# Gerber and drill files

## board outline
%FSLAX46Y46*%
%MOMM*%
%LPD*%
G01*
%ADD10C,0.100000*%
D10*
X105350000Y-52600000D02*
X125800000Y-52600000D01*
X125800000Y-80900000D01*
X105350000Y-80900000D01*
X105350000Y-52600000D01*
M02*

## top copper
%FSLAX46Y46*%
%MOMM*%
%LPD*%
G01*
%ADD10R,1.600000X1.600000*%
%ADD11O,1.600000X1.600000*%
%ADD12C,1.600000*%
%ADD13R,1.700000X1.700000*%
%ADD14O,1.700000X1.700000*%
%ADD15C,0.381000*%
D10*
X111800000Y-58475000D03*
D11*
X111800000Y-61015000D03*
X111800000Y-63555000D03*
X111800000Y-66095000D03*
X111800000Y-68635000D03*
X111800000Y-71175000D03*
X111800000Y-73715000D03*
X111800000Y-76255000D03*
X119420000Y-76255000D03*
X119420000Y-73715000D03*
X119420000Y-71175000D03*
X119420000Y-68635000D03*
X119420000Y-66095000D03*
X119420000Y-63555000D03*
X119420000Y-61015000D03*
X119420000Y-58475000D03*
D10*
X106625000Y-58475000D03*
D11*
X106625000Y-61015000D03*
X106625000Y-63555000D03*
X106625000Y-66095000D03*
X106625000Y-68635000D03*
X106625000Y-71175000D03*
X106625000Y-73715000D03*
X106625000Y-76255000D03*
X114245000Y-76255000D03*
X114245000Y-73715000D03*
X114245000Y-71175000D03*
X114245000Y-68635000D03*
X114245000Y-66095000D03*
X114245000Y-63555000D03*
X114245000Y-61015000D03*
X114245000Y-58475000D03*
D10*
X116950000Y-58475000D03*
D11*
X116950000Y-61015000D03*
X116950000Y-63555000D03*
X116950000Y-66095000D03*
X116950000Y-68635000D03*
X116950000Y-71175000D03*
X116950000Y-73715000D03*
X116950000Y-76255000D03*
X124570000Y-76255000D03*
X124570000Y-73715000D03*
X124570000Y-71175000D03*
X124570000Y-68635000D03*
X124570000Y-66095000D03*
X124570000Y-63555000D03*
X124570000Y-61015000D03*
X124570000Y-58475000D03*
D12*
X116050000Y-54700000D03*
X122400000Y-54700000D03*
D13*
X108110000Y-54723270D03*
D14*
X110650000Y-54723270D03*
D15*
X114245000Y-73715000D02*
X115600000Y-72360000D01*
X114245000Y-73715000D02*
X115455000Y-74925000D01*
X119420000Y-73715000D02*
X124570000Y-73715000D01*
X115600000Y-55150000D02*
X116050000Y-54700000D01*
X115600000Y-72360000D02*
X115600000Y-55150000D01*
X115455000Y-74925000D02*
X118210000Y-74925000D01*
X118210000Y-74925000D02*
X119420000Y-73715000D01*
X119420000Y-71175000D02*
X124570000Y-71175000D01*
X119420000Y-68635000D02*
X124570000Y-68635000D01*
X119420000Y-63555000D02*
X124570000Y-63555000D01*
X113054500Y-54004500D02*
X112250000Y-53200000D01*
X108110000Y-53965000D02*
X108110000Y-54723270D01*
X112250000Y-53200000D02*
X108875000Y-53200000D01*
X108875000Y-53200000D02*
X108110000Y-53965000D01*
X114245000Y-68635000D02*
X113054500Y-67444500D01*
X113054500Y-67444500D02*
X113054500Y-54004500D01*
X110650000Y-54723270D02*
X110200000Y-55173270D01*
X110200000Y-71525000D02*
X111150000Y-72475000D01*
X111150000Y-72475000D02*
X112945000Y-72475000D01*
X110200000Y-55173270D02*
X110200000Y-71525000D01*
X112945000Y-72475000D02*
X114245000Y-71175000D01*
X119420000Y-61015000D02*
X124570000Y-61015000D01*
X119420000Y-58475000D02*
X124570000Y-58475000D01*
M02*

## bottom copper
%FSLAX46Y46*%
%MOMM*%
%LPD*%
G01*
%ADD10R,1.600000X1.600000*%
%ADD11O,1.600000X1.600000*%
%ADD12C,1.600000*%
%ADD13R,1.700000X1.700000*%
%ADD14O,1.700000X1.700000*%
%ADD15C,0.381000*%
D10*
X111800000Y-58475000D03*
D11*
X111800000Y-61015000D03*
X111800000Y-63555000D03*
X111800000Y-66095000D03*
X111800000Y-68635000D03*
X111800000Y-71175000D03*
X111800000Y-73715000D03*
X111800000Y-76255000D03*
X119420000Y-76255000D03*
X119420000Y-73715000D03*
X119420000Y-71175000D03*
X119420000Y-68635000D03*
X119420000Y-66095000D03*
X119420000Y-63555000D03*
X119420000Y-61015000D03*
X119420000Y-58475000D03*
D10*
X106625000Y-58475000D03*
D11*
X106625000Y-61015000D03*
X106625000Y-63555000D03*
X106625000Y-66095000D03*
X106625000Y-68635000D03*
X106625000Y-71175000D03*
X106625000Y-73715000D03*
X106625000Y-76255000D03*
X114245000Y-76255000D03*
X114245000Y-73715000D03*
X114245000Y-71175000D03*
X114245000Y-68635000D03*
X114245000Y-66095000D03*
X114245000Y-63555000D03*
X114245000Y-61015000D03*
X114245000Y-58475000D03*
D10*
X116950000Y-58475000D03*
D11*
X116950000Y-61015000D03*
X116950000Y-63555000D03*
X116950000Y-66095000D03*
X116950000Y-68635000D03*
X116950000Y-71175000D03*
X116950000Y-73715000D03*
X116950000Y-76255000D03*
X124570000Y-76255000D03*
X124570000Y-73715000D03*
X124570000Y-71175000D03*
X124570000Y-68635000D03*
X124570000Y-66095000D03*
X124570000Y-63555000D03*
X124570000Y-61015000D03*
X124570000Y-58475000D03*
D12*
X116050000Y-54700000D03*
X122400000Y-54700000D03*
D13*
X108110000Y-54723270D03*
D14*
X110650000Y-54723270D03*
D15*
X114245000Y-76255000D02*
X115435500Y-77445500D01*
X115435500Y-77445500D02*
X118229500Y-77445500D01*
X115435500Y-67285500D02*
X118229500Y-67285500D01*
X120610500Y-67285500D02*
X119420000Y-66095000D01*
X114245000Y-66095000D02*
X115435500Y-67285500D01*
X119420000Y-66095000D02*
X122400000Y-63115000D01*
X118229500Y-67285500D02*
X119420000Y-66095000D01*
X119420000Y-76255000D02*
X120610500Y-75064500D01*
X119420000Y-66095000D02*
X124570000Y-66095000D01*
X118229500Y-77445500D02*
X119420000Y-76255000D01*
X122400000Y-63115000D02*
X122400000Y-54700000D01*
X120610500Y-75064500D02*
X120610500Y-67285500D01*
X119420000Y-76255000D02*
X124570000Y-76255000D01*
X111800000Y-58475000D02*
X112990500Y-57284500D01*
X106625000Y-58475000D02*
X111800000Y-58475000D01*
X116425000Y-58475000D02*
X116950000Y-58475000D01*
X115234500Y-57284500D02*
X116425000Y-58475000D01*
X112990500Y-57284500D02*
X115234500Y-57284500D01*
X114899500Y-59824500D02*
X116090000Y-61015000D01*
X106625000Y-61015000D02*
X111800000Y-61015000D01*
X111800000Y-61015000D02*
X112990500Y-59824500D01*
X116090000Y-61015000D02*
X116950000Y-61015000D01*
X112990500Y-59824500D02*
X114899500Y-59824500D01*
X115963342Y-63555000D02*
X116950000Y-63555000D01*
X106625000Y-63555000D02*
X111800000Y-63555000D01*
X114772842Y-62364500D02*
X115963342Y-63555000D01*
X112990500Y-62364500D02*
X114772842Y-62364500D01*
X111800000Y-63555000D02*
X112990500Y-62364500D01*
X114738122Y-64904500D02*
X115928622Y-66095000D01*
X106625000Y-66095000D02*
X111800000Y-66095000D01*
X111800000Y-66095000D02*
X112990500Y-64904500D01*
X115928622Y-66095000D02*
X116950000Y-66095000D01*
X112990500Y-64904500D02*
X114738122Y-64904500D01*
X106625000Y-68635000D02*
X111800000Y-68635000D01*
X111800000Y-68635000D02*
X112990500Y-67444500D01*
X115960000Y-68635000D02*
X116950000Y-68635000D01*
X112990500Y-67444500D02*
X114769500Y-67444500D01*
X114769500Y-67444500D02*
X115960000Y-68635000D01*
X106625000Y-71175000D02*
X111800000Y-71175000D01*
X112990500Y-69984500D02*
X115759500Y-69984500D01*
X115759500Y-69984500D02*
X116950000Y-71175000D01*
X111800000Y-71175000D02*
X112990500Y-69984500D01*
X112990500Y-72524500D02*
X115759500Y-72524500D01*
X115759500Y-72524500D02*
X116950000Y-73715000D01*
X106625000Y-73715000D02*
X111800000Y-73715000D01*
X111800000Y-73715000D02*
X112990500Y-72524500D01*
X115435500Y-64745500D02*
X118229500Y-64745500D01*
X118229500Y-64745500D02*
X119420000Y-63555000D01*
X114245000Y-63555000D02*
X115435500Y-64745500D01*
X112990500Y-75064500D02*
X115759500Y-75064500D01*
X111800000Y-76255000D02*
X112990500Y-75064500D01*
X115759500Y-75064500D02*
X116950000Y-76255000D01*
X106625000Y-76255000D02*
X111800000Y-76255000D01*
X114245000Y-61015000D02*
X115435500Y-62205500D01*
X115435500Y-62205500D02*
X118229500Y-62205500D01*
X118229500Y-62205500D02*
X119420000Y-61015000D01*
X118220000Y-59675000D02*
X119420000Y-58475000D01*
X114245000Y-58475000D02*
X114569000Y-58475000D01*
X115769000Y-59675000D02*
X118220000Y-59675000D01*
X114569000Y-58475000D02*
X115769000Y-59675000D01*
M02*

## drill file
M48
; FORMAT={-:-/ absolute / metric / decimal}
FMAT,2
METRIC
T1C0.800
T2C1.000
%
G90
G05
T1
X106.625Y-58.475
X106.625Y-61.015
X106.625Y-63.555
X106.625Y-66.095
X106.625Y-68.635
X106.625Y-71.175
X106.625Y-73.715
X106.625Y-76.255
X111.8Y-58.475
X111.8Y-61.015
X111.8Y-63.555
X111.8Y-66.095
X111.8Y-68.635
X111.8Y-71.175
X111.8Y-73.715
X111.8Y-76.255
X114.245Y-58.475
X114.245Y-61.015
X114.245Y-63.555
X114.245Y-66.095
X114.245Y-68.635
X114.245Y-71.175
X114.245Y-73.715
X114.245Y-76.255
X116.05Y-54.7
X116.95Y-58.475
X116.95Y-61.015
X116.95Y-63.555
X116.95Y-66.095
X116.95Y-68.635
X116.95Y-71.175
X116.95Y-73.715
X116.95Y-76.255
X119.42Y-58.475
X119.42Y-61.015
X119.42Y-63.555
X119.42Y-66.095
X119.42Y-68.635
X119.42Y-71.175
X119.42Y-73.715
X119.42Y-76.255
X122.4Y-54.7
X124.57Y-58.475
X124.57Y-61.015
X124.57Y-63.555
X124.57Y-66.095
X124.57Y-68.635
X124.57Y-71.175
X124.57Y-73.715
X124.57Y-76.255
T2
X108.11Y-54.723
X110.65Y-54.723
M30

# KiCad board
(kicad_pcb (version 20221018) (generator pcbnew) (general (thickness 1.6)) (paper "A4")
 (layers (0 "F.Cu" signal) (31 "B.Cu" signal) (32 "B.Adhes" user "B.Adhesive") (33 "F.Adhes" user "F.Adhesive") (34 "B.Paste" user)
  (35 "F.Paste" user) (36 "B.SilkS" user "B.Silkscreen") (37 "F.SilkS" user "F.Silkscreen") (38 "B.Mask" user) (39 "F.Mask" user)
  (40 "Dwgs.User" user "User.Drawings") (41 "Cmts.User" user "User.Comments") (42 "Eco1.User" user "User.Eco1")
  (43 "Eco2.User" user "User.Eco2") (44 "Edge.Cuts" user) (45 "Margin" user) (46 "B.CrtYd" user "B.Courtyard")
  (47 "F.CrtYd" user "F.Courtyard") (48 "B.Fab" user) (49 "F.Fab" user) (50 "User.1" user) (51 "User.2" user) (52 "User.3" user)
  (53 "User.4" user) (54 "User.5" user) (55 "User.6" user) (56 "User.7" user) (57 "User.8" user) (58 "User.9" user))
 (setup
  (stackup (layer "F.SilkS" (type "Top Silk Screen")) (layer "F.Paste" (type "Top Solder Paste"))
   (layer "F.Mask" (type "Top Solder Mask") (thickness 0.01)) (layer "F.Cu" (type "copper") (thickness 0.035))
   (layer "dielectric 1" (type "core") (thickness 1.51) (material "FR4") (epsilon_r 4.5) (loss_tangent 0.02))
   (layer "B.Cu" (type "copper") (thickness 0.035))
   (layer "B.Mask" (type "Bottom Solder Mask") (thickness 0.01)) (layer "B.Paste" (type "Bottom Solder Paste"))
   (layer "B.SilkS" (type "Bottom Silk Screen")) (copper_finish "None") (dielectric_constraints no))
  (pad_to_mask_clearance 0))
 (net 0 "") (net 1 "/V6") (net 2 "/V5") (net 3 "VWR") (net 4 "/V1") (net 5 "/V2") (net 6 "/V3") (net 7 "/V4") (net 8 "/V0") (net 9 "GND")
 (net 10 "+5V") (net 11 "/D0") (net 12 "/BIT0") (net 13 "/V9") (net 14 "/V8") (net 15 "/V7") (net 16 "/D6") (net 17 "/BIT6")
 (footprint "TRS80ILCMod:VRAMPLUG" (layer "F.Cu") (at 111.8 58.475)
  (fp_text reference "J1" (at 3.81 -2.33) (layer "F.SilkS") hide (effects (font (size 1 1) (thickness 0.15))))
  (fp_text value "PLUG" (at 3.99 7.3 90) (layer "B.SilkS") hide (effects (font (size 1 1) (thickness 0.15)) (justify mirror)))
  (pad "1" thru_hole rect (at 0 0) (size 1.6 1.6) (drill 0.8) (layers "*.Cu" "*.Mask") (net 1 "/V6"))
  (pad "2" thru_hole oval (at 0 2.54) (size 1.6 1.6) (drill 0.8) (layers "*.Cu" "*.Mask") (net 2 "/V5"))
  (pad "3" thru_hole oval (at 0 5.08) (size 1.6 1.6) (drill 0.8) (layers "*.Cu" "*.Mask") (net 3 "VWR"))
  (pad "4" thru_hole oval (at 0 7.62) (size 1.6 1.6) (drill 0.8) (layers "*.Cu" "*.Mask") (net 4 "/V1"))
  (pad "5" thru_hole oval (at 0 10.16) (size 1.6 1.6) (drill 0.8) (layers "*.Cu" "*.Mask") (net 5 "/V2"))
  (pad "6" thru_hole oval (at 0 12.7) (size 1.6 1.6) (drill 0.8) (layers "*.Cu" "*.Mask") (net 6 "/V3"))
  (pad "7" thru_hole oval (at 0 15.24) (size 1.6 1.6) (drill 0.8) (layers "*.Cu" "*.Mask") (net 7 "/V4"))
  (pad "8" thru_hole oval (at 0 17.78) (size 1.6 1.6) (drill 0.8) (layers "*.Cu" "*.Mask") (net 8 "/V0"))
  (pad "9" thru_hole oval (at 7.62 17.78) (size 1.6 1.6) (drill 0.8) (layers "*.Cu" "*.Mask") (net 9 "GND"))
  (pad "10" thru_hole oval (at 7.62 15.24) (size 1.6 1.6) (drill 0.8) (layers "*.Cu" "*.Mask") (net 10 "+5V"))
  (pad "11" thru_hole oval (at 7.62 12.7) (size 1.6 1.6) (drill 0.8) (layers "*.Cu" "*.Mask") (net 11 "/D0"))
  (pad "12" thru_hole oval (at 7.62 10.16) (size 1.6 1.6) (drill 0.8) (layers "*.Cu" "*.Mask") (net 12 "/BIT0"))
  (pad "13" thru_hole oval (at 7.62 7.62) (size 1.6 1.6) (drill 0.8) (layers "*.Cu" "*.Mask") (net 9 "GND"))
  (pad "14" thru_hole oval (at 7.62 5.08) (size 1.6 1.6) (drill 0.8) (layers "*.Cu" "*.Mask") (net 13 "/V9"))
  (pad "15" thru_hole oval (at 7.62 2.54) (size 1.6 1.6) (drill 0.8) (layers "*.Cu" "*.Mask") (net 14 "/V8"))
  (pad "16" thru_hole oval (at 7.62 0) (size 1.6 1.6) (drill 0.8) (layers "*.Cu" "*.Mask") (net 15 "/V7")))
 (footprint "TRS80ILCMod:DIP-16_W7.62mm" (layer "F.Cu") (at 106.625 58.475)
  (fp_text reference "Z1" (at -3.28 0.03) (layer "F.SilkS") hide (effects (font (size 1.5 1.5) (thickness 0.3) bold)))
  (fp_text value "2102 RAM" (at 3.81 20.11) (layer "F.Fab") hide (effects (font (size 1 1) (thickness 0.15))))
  (pad "1" thru_hole rect (at 0 0) (size 1.6 1.6) (drill 0.8) (layers "*.Cu" "*.Mask") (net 1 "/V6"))
  (pad "2" thru_hole oval (at 0 2.54) (size 1.6 1.6) (drill 0.8) (layers "*.Cu" "*.Mask") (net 2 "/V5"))
  (pad "3" thru_hole oval (at 0 5.08) (size 1.6 1.6) (drill 0.8) (layers "*.Cu" "*.Mask") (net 3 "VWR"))
  (pad "4" thru_hole oval (at 0 7.62) (size 1.6 1.6) (drill 0.8) (layers "*.Cu" "*.Mask") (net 4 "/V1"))
  (pad "5" thru_hole oval (at 0 10.16) (size 1.6 1.6) (drill 0.8) (layers "*.Cu" "*.Mask") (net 5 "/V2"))
  (pad "6" thru_hole oval (at 0 12.7) (size 1.6 1.6) (drill 0.8) (layers "*.Cu" "*.Mask") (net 6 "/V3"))
  (pad "7" thru_hole oval (at 0 15.24) (size 1.6 1.6) (drill 0.8) (layers "*.Cu" "*.Mask") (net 7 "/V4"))
  (pad "8" thru_hole oval (at 0 17.78) (size 1.6 1.6) (drill 0.8) (layers "*.Cu" "*.Mask") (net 8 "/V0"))
  (pad "9" thru_hole oval (at 7.62 17.78) (size 1.6 1.6) (drill 0.8) (layers "*.Cu" "*.Mask") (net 9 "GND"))
  (pad "10" thru_hole oval (at 7.62 15.24) (size 1.6 1.6) (drill 0.8) (layers "*.Cu" "*.Mask") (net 10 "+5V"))
  (pad "11" thru_hole oval (at 7.62 12.7) (size 1.6 1.6) (drill 0.8) (layers "*.Cu" "*.Mask") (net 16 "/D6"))
  (pad "12" thru_hole oval (at 7.62 10.16) (size 1.6 1.6) (drill 0.8) (layers "*.Cu" "*.Mask") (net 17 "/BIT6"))
  (pad "13" thru_hole oval (at 7.62 7.62) (size 1.6 1.6) (drill 0.8) (layers "*.Cu" "*.Mask") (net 9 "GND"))
  (pad "14" thru_hole oval (at 7.62 5.08) (size 1.6 1.6) (drill 0.8) (layers "*.Cu" "*.Mask") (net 13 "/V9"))
  (pad "15" thru_hole oval (at 7.62 2.54) (size 1.6 1.6) (drill 0.8) (layers "*.Cu" "*.Mask") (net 14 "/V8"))
  (pad "16" thru_hole oval (at 7.62 0) (size 1.6 1.6) (drill 0.8) (layers "*.Cu" "*.Mask") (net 15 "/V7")))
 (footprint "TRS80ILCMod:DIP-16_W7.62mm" (layer "F.Cu") (at 116.95 58.475)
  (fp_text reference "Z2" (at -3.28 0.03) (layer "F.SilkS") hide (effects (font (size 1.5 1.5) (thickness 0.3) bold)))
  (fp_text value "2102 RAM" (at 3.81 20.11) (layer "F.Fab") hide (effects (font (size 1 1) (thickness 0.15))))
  (pad "1" thru_hole rect (at 0 0) (size 1.6 1.6) (drill 0.8) (layers "*.Cu" "*.Mask") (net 1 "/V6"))
  (pad "2" thru_hole oval (at 0 2.54) (size 1.6 1.6) (drill 0.8) (layers "*.Cu" "*.Mask") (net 2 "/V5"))
  (pad "3" thru_hole oval (at 0 5.08) (size 1.6 1.6) (drill 0.8) (layers "*.Cu" "*.Mask") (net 3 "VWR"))
  (pad "4" thru_hole oval (at 0 7.62) (size 1.6 1.6) (drill 0.8) (layers "*.Cu" "*.Mask") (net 4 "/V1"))
  (pad "5" thru_hole oval (at 0 10.16) (size 1.6 1.6) (drill 0.8) (layers "*.Cu" "*.Mask") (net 5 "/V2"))
  (pad "6" thru_hole oval (at 0 12.7) (size 1.6 1.6) (drill 0.8) (layers "*.Cu" "*.Mask") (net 6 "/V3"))
  (pad "7" thru_hole oval (at 0 15.24) (size 1.6 1.6) (drill 0.8) (layers "*.Cu" "*.Mask") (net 7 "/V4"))
  (pad "8" thru_hole oval (at 0 17.78) (size 1.6 1.6) (drill 0.8) (layers "*.Cu" "*.Mask") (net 8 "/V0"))
  (pad "9" thru_hole oval (at 7.62 17.78) (size 1.6 1.6) (drill 0.8) (layers "*.Cu" "*.Mask") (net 9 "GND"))
  (pad "10" thru_hole oval (at 7.62 15.24) (size 1.6 1.6) (drill 0.8) (layers "*.Cu" "*.Mask") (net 10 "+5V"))
  (pad "11" thru_hole oval (at 7.62 12.7) (size 1.6 1.6) (drill 0.8) (layers "*.Cu" "*.Mask") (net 11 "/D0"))
  (pad "12" thru_hole oval (at 7.62 10.16) (size 1.6 1.6) (drill 0.8) (layers "*.Cu" "*.Mask") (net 12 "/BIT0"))
  (pad "13" thru_hole oval (at 7.62 7.62) (size 1.6 1.6) (drill 0.8) (layers "*.Cu" "*.Mask") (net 9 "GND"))
  (pad "14" thru_hole oval (at 7.62 5.08) (size 1.6 1.6) (drill 0.8) (layers "*.Cu" "*.Mask") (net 13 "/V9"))
  (pad "15" thru_hole oval (at 7.62 2.54) (size 1.6 1.6) (drill 0.8) (layers "*.Cu" "*.Mask") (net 14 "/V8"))
  (pad "16" thru_hole oval (at 7.62 0) (size 1.6 1.6) (drill 0.8) (layers "*.Cu" "*.Mask") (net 15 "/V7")))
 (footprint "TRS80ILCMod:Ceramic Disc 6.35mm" (layer "F.Cu") (at 115.69 54.71)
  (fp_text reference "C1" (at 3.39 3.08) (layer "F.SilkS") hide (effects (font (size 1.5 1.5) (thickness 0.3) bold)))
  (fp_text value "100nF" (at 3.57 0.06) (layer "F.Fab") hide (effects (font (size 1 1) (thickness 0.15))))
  (pad "1" thru_hole circle (at 0.36 -0.01) (size 1.6 1.6) (drill 0.8) (layers "*.Cu" "*.Mask") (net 10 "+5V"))
  (pad "2" thru_hole circle (at 6.71 -0.01) (size 1.6 1.6) (drill 0.8) (layers "*.Cu" "*.Mask") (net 9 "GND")))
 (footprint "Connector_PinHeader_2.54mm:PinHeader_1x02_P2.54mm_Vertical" (layer "F.Cu") (at 108.11 54.72327 90)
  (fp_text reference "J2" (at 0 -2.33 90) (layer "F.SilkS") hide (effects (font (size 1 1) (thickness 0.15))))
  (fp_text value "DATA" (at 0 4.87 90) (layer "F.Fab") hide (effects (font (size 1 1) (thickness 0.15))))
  (pad "1" thru_hole rect (at 0 0 90) (size 1.7 1.7) (drill 1) (layers "*.Cu" "*.Mask") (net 17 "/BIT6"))
  (pad "2" thru_hole oval (at 0 2.54 90) (size 1.7 1.7) (drill 1) (layers "*.Cu" "*.Mask") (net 16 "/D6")))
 (gr_rect (start 105.35 52.6) (end 125.8 80.9) (stroke (width 0.1) (type default)) (fill none) (layer "Edge.Cuts"))
 (segment (start 114.245 76.255) (end 115.4355 77.4455) (width 0.381) (layer "B.Cu") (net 9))
 (segment (start 115.4355 77.4455) (end 118.2295 77.4455) (width 0.381) (layer "B.Cu") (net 9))
 (segment (start 115.4355 67.2855) (end 118.2295 67.2855) (width 0.381) (layer "B.Cu") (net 9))
 (segment (start 120.6105 67.2855) (end 119.42 66.095) (width 0.381) (layer "B.Cu") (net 9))
 (segment (start 114.245 66.095) (end 115.4355 67.2855) (width 0.381) (layer "B.Cu") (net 9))
 (segment (start 119.42 66.095) (end 122.4 63.115) (width 0.381) (layer "B.Cu") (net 9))
 (segment (start 118.2295 67.2855) (end 119.42 66.095) (width 0.381) (layer "B.Cu") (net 9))
 (segment (start 119.42 76.255) (end 120.6105 75.0645) (width 0.381) (layer "B.Cu") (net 9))
 (segment (start 119.42 66.095) (end 124.57 66.095) (width 0.381) (layer "B.Cu") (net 9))
 (segment (start 118.2295 77.4455) (end 119.42 76.255) (width 0.381) (layer "B.Cu") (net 9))
 (segment (start 122.4 63.115) (end 122.4 54.7) (width 0.381) (layer "B.Cu") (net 9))
 (segment (start 120.6105 75.0645) (end 120.6105 67.2855) (width 0.381) (layer "B.Cu") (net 9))
 (segment (start 119.42 76.255) (end 124.57 76.255) (width 0.381) (layer "B.Cu") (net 9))
 (segment (start 114.245 73.715) (end 115.6 72.36) (width 0.381) (layer "F.Cu") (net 10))
 (segment (start 114.245 73.715) (end 115.455 74.925) (width 0.381) (layer "F.Cu") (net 10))
 (segment (start 119.42 73.715) (end 124.57 73.715) (width 0.381) (layer "F.Cu") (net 10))
 (segment (start 115.6 55.15) (end 116.05 54.7) (width 0.381) (layer "F.Cu") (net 10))
 (segment (start 115.6 72.36) (end 115.6 55.15) (width 0.381) (layer "F.Cu") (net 10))
 (segment (start 115.455 74.925) (end 118.21 74.925) (width 0.381) (layer "F.Cu") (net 10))
 (segment (start 118.21 74.925) (end 119.42 73.715) (width 0.381) (layer "F.Cu") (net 10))
 (segment (start 111.8 58.475) (end 112.9905 57.2845) (width 0.381) (layer "B.Cu") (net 1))
 (segment (start 106.625 58.475) (end 111.8 58.475) (width 0.381) (layer "B.Cu") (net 1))
 (segment (start 116.425 58.475) (end 116.95 58.475) (width 0.381) (layer "B.Cu") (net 1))
 (segment (start 115.2345 57.2845) (end 116.425 58.475) (width 0.381) (layer "B.Cu") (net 1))
 (segment (start 112.9905 57.2845) (end 115.2345 57.2845) (width 0.381) (layer "B.Cu") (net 1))
 (segment (start 114.8995 59.8245) (end 116.09 61.015) (width 0.381) (layer "B.Cu") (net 2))
 (segment (start 106.625 61.015) (end 111.8 61.015) (width 0.381) (layer "B.Cu") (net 2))
 (segment (start 111.8 61.015) (end 112.9905 59.8245) (width 0.381) (layer "B.Cu") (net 2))
 (segment (start 116.09 61.015) (end 116.95 61.015) (width 0.381) (layer "B.Cu") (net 2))
 (segment (start 112.9905 59.8245) (end 114.8995 59.8245) (width 0.381) (layer "B.Cu") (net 2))
 (segment (start 115.963342 63.555) (end 116.95 63.555) (width 0.381) (layer "B.Cu") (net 3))
 (segment (start 106.625 63.555) (end 111.8 63.555) (width 0.381) (layer "B.Cu") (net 3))
 (segment (start 114.772842 62.3645) (end 115.963342 63.555) (width 0.381) (layer "B.Cu") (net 3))
 (segment (start 112.9905 62.3645) (end 114.772842 62.3645) (width 0.381) (layer "B.Cu") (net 3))
 (segment (start 111.8 63.555) (end 112.9905 62.3645) (width 0.381) (layer "B.Cu") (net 3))
 (segment (start 114.738122 64.9045) (end 115.928622 66.095) (width 0.381) (layer "B.Cu") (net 4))
 (segment (start 106.625 66.095) (end 111.8 66.095) (width 0.381) (layer "B.Cu") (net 4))
 (segment (start 111.8 66.095) (end 112.9905 64.9045) (width 0.381) (layer "B.Cu") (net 4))
 (segment (start 115.928622 66.095) (end 116.95 66.095) (width 0.381) (layer "B.Cu") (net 4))
 (segment (start 112.9905 64.9045) (end 114.738122 64.9045) (width 0.381) (layer "B.Cu") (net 4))
 (segment (start 106.625 68.635) (end 111.8 68.635) (width 0.381) (layer "B.Cu") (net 5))
 (segment (start 111.8 68.635) (end 112.9905 67.4445) (width 0.381) (layer "B.Cu") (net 5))
 (segment (start 115.96 68.635) (end 116.95 68.635) (width 0.381) (layer "B.Cu") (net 5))
 (segment (start 112.9905 67.4445) (end 114.7695 67.4445) (width 0.381) (layer "B.Cu") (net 5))
 (segment (start 114.7695 67.4445) (end 115.96 68.635) (width 0.381) (layer "B.Cu") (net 5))
 (segment (start 106.625 71.175) (end 111.8 71.175) (width 0.381) (layer "B.Cu") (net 6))
 (segment (start 112.9905 69.9845) (end 115.7595 69.9845) (width 0.381) (layer "B.Cu") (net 6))
 (segment (start 115.7595 69.9845) (end 116.95 71.175) (width 0.381) (layer "B.Cu") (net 6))
 (segment (start 111.8 71.175) (end 112.9905 69.9845) (width 0.381) (layer "B.Cu") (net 6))
 (segment (start 112.9905 72.5245) (end 115.7595 72.5245) (width 0.381) (layer "B.Cu") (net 7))
 (segment (start 115.7595 72.5245) (end 116.95 73.715) (width 0.381) (layer "B.Cu") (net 7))
 (segment (start 106.625 73.715) (end 111.8 73.715) (width 0.381) (layer "B.Cu") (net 7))
 (segment (start 111.8 73.715) (end 112.9905 72.5245) (width 0.381) (layer "B.Cu") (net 7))
 (segment (start 119.42 71.175) (end 124.57 71.175) (width 0.381) (layer "F.Cu") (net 11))
 (segment (start 119.42 68.635) (end 124.57 68.635) (width 0.381) (layer "F.Cu") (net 12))
 (segment (start 119.42 63.555) (end 124.57 63.555) (width 0.381) (layer "F.Cu") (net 13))
 (segment (start 115.4355 64.7455) (end 118.2295 64.7455) (width 0.381) (layer "B.Cu") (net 13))
 (segment (start 118.2295 64.7455) (end 119.42 63.555) (width 0.381) (layer "B.Cu") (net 13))
 (segment (start 114.245 63.555) (end 115.4355 64.7455) (width 0.381) (layer "B.Cu") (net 13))
 (segment (start 113.0545 54.0045) (end 112.25 53.2) (width 0.381) (layer "F.Cu") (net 17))
 (segment (start 108.11 53.965) (end 108.11 54.72327) (width 0.381) (layer "F.Cu") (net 17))
 (segment (start 112.25 53.2) (end 108.875 53.2) (width 0.381) (layer "F.Cu") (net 17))
 (segment (start 108.875 53.2) (end 108.11 53.965) (width 0.381) (layer "F.Cu") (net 17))
 (segment (start 114.245 68.635) (end 113.0545 67.4445) (width 0.381) (layer "F.Cu") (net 17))
 (segment (start 113.0545 67.4445) (end 113.0545 54.0045) (width 0.381) (layer "F.Cu") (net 17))
 (segment (start 110.65 54.72327) (end 110.2 55.17327) (width 0.381) (layer "F.Cu") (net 16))
 (segment (start 110.2 71.525) (end 111.15 72.475) (width 0.381) (layer "F.Cu") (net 16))
 (segment (start 111.15 72.475) (end 112.945 72.475) (width 0.381) (layer "F.Cu") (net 16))
 (segment (start 110.2 55.17327) (end 110.2 71.525) (width 0.381) (layer "F.Cu") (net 16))
 (segment (start 112.945 72.475) (end 114.245 71.175) (width 0.381) (layer "F.Cu") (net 16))
 (segment (start 112.9905 75.0645) (end 115.7595 75.0645) (width 0.381) (layer "B.Cu") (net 8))
 (segment (start 111.8 76.255) (end 112.9905 75.0645) (width 0.381) (layer "B.Cu") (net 8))
 (segment (start 115.7595 75.0645) (end 116.95 76.255) (width 0.381) (layer "B.Cu") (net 8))
 (segment (start 106.625 76.255) (end 111.8 76.255) (width 0.381) (layer "B.Cu") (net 8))
 (segment (start 119.42 61.015) (end 124.57 61.015) (width 0.381) (layer "F.Cu") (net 14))
 (segment (start 114.245 61.015) (end 115.4355 62.2055) (width 0.381) (layer "B.Cu") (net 14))
 (segment (start 115.4355 62.2055) (end 118.2295 62.2055) (width 0.381) (layer "B.Cu") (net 14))
 (segment (start 118.2295 62.2055) (end 119.42 61.015) (width 0.381) (layer "B.Cu") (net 14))
 (segment (start 119.42 58.475) (end 124.57 58.475) (width 0.381) (layer "F.Cu") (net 15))
 (segment (start 118.22 59.675) (end 119.42 58.475) (width 0.381) (layer "B.Cu") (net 15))
 (segment (start 114.245 58.475) (end 114.569 58.475) (width 0.381) (layer "B.Cu") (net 15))
 (segment (start 115.769 59.675) (end 118.22 59.675) (width 0.381) (layer "B.Cu") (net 15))
 (segment (start 114.569 58.475) (end 115.769 59.675) (width 0.381) (layer "B.Cu") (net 15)))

